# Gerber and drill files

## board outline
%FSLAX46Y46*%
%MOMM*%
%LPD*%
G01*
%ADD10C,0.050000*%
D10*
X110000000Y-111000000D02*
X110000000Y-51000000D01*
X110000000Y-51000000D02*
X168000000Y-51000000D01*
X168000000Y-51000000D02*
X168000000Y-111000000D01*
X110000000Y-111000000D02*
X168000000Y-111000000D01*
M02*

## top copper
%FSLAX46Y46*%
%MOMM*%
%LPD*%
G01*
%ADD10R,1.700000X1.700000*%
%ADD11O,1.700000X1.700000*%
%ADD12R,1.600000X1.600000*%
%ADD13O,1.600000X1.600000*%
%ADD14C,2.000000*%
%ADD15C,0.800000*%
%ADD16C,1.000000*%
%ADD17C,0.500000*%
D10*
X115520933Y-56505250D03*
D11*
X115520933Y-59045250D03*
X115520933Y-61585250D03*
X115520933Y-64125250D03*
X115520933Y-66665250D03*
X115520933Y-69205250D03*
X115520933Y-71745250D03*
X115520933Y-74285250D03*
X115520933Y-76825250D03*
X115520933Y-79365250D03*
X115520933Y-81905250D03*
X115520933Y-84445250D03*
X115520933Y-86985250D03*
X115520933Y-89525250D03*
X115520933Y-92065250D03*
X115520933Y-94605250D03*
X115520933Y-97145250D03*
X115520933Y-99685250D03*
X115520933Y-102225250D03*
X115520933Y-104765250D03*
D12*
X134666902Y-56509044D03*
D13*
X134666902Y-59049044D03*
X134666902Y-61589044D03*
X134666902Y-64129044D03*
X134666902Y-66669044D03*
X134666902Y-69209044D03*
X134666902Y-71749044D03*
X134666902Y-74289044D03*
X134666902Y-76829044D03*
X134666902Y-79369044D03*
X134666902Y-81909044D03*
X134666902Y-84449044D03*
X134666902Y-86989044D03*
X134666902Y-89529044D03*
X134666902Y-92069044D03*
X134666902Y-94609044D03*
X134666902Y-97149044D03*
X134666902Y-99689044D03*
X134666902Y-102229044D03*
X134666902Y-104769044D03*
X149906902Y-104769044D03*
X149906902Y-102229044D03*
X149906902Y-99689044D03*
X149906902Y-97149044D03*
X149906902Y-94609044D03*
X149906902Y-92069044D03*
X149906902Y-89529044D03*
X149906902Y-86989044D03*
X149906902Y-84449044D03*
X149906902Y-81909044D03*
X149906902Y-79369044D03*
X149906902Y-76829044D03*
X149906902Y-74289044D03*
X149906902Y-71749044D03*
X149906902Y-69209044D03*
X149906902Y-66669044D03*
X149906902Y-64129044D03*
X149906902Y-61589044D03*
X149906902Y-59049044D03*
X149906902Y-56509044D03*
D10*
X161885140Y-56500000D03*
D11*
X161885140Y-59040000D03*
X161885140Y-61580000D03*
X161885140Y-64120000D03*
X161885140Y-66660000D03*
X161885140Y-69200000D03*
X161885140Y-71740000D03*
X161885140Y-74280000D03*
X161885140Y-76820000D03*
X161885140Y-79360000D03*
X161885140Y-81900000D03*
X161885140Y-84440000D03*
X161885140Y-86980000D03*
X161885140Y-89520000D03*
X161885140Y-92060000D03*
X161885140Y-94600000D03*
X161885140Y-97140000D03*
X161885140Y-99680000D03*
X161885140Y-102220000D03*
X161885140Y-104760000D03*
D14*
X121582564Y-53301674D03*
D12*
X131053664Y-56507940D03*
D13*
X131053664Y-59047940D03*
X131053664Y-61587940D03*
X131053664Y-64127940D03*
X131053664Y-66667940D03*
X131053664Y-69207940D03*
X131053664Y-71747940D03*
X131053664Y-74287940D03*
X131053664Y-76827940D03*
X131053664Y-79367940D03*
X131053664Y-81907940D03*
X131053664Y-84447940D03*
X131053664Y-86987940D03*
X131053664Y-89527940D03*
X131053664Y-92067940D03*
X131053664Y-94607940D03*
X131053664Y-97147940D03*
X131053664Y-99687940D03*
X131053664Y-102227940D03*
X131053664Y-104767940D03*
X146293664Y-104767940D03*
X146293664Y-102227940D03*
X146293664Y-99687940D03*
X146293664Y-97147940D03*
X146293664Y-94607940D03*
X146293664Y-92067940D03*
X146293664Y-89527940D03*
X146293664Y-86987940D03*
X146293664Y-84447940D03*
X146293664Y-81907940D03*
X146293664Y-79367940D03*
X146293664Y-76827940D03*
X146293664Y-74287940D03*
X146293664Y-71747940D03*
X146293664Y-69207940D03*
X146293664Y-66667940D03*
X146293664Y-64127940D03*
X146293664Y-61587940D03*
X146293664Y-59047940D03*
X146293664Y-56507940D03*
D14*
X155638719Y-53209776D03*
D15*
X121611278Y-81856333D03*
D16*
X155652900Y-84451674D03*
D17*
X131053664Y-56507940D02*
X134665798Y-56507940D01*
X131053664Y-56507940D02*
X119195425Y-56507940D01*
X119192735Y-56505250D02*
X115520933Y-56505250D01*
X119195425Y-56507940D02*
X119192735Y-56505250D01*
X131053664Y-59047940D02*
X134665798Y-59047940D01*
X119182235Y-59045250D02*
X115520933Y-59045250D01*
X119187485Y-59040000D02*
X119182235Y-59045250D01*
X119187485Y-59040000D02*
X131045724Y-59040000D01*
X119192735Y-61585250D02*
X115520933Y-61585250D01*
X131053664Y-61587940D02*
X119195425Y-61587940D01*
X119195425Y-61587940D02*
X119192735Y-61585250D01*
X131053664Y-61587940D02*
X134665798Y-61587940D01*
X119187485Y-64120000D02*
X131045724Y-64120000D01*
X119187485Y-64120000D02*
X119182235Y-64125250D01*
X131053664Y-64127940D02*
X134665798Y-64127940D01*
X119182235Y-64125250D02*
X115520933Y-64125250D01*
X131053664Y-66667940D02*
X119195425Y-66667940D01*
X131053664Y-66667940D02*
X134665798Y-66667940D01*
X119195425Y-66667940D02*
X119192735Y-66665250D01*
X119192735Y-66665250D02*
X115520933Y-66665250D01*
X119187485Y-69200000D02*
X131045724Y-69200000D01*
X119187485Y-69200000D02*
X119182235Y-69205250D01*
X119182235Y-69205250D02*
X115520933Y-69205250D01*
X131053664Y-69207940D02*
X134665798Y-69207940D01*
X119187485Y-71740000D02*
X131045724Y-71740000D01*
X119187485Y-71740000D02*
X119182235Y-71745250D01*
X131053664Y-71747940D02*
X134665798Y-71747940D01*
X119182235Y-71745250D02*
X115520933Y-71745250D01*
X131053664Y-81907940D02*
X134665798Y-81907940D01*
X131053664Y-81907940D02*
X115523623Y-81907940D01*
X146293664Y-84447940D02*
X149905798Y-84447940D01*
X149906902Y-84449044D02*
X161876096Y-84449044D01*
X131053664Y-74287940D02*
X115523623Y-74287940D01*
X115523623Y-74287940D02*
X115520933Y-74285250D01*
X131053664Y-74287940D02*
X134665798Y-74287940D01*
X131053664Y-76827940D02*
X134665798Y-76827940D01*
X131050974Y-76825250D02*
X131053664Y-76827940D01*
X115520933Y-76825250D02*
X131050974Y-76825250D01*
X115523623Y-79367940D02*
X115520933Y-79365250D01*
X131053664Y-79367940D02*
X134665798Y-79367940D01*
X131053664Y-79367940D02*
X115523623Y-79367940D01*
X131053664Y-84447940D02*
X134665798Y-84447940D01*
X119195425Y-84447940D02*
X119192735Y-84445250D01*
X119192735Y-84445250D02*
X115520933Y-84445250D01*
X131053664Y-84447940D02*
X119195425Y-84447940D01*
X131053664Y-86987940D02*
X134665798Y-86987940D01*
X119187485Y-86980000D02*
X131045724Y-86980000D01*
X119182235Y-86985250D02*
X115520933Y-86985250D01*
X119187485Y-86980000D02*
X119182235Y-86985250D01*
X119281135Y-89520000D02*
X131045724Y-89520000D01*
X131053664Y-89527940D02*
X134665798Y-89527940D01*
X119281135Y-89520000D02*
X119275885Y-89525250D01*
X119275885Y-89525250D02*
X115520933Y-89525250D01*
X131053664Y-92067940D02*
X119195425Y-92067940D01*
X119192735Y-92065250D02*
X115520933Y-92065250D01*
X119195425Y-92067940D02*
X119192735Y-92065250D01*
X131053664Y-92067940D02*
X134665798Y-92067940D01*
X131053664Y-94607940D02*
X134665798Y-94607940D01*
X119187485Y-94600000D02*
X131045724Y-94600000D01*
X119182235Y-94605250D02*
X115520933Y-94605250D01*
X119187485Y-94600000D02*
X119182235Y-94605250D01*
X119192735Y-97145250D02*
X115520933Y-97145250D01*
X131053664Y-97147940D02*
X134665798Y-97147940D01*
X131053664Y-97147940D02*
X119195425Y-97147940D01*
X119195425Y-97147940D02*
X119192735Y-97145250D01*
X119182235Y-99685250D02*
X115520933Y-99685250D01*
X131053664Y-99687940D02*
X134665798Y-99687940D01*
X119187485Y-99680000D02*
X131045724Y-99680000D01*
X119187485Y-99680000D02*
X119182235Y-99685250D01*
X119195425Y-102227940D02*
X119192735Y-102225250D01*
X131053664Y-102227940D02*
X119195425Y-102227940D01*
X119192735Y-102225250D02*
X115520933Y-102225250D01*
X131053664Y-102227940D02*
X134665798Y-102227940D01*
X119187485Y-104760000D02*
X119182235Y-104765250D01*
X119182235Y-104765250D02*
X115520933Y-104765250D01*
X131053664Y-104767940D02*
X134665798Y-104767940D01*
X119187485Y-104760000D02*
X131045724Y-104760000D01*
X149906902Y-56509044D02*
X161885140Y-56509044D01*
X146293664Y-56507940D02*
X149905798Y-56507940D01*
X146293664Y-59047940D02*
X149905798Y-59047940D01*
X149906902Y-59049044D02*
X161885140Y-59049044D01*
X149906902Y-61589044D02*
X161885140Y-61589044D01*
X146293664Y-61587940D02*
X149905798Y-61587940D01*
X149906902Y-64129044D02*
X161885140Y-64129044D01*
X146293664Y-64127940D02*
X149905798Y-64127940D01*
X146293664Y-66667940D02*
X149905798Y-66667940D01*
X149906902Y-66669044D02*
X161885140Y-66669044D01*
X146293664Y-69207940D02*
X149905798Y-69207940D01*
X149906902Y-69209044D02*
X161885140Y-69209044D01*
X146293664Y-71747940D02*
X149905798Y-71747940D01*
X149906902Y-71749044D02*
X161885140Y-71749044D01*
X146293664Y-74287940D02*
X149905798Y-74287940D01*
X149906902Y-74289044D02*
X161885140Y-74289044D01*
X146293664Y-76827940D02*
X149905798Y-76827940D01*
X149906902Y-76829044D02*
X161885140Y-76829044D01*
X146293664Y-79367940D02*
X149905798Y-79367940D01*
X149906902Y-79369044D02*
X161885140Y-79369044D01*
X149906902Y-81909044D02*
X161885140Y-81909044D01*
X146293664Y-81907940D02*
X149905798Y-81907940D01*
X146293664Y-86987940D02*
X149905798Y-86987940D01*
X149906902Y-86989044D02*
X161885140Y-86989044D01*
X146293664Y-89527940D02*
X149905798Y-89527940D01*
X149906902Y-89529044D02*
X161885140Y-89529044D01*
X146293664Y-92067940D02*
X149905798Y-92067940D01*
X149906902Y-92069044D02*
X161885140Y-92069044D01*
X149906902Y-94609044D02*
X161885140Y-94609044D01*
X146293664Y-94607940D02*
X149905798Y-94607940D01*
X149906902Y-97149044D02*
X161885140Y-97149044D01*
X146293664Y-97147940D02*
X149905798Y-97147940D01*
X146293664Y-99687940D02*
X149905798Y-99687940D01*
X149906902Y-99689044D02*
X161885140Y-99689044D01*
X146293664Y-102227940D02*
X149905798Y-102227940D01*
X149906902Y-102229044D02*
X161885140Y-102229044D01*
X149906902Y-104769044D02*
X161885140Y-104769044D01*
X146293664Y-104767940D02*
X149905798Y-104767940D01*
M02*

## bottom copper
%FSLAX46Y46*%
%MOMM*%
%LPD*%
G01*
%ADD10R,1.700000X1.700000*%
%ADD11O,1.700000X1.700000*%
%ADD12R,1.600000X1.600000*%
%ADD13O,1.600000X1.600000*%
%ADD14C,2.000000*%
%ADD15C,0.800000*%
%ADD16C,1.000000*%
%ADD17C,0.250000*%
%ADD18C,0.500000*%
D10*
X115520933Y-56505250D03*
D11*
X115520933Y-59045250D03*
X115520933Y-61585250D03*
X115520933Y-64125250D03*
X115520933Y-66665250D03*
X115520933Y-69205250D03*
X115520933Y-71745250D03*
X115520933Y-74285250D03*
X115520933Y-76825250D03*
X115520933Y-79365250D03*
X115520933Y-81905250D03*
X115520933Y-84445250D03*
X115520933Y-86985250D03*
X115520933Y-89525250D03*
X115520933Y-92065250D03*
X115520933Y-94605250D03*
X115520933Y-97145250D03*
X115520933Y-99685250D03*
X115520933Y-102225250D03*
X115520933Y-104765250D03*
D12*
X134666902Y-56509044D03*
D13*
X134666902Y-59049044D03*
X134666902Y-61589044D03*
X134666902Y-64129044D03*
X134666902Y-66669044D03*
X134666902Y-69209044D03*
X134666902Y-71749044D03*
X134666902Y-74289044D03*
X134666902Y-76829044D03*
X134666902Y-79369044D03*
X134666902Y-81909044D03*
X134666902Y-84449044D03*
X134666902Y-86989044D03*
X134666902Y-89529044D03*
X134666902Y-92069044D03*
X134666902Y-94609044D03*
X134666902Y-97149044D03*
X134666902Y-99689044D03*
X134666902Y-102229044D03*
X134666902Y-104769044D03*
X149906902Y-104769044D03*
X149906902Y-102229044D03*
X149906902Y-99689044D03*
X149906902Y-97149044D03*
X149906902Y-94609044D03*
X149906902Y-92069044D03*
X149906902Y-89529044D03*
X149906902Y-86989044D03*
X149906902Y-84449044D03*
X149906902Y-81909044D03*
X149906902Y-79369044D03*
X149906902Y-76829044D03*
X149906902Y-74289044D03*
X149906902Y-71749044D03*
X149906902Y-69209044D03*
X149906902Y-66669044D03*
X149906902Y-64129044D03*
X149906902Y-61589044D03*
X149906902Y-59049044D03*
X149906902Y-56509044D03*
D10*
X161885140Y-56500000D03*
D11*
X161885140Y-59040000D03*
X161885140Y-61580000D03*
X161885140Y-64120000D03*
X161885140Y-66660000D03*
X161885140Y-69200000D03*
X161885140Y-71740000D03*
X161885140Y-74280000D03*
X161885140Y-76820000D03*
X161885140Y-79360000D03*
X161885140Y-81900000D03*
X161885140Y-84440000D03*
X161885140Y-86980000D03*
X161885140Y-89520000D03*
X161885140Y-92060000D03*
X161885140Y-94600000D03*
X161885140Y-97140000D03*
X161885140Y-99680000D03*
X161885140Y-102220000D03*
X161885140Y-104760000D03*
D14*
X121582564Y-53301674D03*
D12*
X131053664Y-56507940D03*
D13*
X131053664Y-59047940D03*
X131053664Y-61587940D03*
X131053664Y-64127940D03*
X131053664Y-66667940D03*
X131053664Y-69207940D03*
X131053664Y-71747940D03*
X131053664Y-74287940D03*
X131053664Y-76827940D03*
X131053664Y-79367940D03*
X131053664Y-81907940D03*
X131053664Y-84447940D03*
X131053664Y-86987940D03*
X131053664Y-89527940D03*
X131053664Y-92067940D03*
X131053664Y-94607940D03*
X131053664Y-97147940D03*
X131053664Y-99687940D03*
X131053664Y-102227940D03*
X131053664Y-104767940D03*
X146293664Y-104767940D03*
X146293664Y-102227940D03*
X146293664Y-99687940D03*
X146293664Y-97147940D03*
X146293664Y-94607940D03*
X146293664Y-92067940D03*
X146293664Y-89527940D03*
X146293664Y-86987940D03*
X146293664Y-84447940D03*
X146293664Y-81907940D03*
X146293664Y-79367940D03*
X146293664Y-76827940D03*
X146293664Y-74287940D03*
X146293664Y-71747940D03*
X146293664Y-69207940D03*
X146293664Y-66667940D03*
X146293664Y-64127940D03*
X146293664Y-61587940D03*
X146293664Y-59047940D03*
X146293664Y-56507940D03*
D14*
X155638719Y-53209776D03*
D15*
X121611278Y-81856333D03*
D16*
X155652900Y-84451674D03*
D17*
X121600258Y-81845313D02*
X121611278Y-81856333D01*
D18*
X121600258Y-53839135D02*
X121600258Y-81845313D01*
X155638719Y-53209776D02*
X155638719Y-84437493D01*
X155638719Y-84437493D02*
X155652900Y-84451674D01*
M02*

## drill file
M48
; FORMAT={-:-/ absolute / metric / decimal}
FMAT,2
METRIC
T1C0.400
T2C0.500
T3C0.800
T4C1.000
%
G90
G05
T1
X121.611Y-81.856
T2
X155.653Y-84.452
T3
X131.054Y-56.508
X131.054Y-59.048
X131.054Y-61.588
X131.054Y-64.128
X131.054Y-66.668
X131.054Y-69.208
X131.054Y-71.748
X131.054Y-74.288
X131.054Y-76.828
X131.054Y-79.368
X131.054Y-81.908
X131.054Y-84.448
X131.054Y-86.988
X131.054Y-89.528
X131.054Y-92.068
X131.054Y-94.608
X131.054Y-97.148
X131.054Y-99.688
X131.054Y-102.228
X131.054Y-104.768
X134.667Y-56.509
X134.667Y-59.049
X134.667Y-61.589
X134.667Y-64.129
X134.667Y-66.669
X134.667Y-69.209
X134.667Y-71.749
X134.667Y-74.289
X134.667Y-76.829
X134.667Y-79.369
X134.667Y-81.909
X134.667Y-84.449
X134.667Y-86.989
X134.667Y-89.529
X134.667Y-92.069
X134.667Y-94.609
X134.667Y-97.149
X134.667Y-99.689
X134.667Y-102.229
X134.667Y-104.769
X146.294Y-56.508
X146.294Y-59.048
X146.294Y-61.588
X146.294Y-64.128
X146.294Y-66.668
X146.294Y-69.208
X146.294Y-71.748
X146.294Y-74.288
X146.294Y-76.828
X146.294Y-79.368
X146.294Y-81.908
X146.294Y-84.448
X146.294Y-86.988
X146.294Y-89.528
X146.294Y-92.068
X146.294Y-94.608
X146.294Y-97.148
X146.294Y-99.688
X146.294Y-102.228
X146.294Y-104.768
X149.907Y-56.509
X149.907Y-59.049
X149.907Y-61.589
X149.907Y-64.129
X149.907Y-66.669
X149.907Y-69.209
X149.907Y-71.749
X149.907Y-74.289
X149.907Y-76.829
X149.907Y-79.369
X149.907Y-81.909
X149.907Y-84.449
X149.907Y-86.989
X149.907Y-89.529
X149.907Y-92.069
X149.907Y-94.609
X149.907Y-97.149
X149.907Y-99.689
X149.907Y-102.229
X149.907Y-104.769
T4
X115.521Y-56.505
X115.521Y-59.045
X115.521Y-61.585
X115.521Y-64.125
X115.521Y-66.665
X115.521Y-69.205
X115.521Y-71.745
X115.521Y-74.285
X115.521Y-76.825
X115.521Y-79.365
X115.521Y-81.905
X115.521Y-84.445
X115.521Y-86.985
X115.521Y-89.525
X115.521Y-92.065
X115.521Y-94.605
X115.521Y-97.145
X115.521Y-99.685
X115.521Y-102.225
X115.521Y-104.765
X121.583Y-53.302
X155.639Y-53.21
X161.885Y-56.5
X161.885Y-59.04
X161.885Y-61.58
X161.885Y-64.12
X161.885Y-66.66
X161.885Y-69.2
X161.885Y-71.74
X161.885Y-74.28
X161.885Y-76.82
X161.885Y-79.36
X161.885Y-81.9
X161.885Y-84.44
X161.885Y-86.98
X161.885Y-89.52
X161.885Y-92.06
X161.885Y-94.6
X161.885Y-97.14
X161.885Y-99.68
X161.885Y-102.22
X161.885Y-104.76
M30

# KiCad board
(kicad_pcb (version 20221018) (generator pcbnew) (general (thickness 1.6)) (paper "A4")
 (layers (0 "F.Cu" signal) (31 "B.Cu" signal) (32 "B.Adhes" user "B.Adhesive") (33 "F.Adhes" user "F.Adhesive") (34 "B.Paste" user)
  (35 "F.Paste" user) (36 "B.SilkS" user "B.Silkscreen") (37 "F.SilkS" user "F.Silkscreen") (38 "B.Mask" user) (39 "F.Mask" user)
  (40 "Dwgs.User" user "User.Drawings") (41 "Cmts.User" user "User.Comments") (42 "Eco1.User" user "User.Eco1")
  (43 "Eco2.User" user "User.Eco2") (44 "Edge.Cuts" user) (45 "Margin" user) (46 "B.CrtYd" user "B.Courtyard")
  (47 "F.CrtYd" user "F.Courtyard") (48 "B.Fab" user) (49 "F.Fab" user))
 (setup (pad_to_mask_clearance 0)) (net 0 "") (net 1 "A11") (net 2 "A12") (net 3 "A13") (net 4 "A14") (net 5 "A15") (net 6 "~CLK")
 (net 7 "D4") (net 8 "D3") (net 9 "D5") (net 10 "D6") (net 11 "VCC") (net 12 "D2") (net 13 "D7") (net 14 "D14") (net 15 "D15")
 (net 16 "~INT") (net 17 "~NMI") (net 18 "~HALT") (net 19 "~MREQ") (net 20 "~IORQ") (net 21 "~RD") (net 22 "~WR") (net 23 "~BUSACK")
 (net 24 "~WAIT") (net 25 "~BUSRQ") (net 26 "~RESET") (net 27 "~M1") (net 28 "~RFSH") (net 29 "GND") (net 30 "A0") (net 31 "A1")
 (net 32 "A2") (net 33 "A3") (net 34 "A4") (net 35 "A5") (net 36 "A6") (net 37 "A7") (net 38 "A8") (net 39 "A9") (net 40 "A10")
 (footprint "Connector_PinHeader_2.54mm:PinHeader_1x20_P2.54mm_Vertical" (layer "F.Cu") (at 115.520933 56.50525)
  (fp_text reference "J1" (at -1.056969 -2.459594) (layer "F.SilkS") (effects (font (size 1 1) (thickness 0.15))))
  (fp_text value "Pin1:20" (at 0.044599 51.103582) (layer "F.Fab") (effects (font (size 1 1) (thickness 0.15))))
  (pad "1" thru_hole rect (at 0 0) (size 1.7 1.7) (drill 1) (layers "*.Cu" "*.Mask") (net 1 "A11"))
  (pad "2" thru_hole oval (at 0 2.54) (size 1.7 1.7) (drill 1) (layers "*.Cu" "*.Mask") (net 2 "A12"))
  (pad "3" thru_hole oval (at 0 5.08) (size 1.7 1.7) (drill 1) (layers "*.Cu" "*.Mask") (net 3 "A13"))
  (pad "4" thru_hole oval (at 0 7.62) (size 1.7 1.7) (drill 1) (layers "*.Cu" "*.Mask") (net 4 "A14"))
  (pad "5" thru_hole oval (at 0 10.16) (size 1.7 1.7) (drill 1) (layers "*.Cu" "*.Mask") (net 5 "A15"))
  (pad "6" thru_hole oval (at 0 12.7) (size 1.7 1.7) (drill 1) (layers "*.Cu" "*.Mask") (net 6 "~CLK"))
  (pad "7" thru_hole oval (at 0 15.24) (size 1.7 1.7) (drill 1) (layers "*.Cu" "*.Mask") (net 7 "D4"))
  (pad "8" thru_hole oval (at 0 17.78) (size 1.7 1.7) (drill 1) (layers "*.Cu" "*.Mask") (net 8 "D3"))
  (pad "9" thru_hole oval (at 0 20.32) (size 1.7 1.7) (drill 1) (layers "*.Cu" "*.Mask") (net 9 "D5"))
  (pad "10" thru_hole oval (at 0 22.86) (size 1.7 1.7) (drill 1) (layers "*.Cu" "*.Mask") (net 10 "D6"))
  (pad "11" thru_hole oval (at 0 25.4) (size 1.7 1.7) (drill 1) (layers "*.Cu" "*.Mask") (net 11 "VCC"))
  (pad "12" thru_hole oval (at 0 27.94) (size 1.7 1.7) (drill 1) (layers "*.Cu" "*.Mask") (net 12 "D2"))
  (pad "13" thru_hole oval (at 0 30.48) (size 1.7 1.7) (drill 1) (layers "*.Cu" "*.Mask") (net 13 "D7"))
  (pad "14" thru_hole oval (at 0 33.02) (size 1.7 1.7) (drill 1) (layers "*.Cu" "*.Mask") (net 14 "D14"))
  (pad "15" thru_hole oval (at 0 35.56) (size 1.7 1.7) (drill 1) (layers "*.Cu" "*.Mask") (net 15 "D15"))
  (pad "16" thru_hole oval (at 0 38.1) (size 1.7 1.7) (drill 1) (layers "*.Cu" "*.Mask") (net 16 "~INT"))
  (pad "17" thru_hole oval (at 0 40.64) (size 1.7 1.7) (drill 1) (layers "*.Cu" "*.Mask") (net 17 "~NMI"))
  (pad "18" thru_hole oval (at 0 43.18) (size 1.7 1.7) (drill 1) (layers "*.Cu" "*.Mask") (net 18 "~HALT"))
  (pad "19" thru_hole oval (at 0 45.72) (size 1.7 1.7) (drill 1) (layers "*.Cu" "*.Mask") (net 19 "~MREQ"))
  (pad "20" thru_hole oval (at 0 48.26) (size 1.7 1.7) (drill 1) (layers "*.Cu" "*.Mask") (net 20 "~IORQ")))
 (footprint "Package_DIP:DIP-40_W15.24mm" (layer "F.Cu") (at 134.666902 56.509044)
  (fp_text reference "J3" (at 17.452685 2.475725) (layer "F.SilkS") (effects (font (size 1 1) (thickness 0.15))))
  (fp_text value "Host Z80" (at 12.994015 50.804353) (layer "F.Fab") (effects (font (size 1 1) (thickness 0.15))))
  (pad "1" thru_hole rect (at 0 0) (size 1.6 1.6) (drill 0.8) (layers "*.Cu" "*.Mask") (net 1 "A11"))
  (pad "2" thru_hole oval (at 0 2.54) (size 1.6 1.6) (drill 0.8) (layers "*.Cu" "*.Mask") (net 2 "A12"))
  (pad "3" thru_hole oval (at 0 5.08) (size 1.6 1.6) (drill 0.8) (layers "*.Cu" "*.Mask") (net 3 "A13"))
  (pad "4" thru_hole oval (at 0 7.62) (size 1.6 1.6) (drill 0.8) (layers "*.Cu" "*.Mask") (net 4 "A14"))
  (pad "5" thru_hole oval (at 0 10.16) (size 1.6 1.6) (drill 0.8) (layers "*.Cu" "*.Mask") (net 5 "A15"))
  (pad "6" thru_hole oval (at 0 12.7) (size 1.6 1.6) (drill 0.8) (layers "*.Cu" "*.Mask") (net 6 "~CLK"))
  (pad "7" thru_hole oval (at 0 15.24) (size 1.6 1.6) (drill 0.8) (layers "*.Cu" "*.Mask") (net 7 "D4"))
  (pad "8" thru_hole oval (at 0 17.78) (size 1.6 1.6) (drill 0.8) (layers "*.Cu" "*.Mask") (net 8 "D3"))
  (pad "9" thru_hole oval (at 0 20.32) (size 1.6 1.6) (drill 0.8) (layers "*.Cu" "*.Mask") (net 9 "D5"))
  (pad "10" thru_hole oval (at 0 22.86) (size 1.6 1.6) (drill 0.8) (layers "*.Cu" "*.Mask") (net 10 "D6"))
  (pad "11" thru_hole oval (at 0 25.4) (size 1.6 1.6) (drill 0.8) (layers "*.Cu" "*.Mask") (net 11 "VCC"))
  (pad "12" thru_hole oval (at 0 27.94) (size 1.6 1.6) (drill 0.8) (layers "*.Cu" "*.Mask") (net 12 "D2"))
  (pad "13" thru_hole oval (at 0 30.48) (size 1.6 1.6) (drill 0.8) (layers "*.Cu" "*.Mask") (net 13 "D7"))
  (pad "14" thru_hole oval (at 0 33.02) (size 1.6 1.6) (drill 0.8) (layers "*.Cu" "*.Mask") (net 14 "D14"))
  (pad "15" thru_hole oval (at 0 35.56) (size 1.6 1.6) (drill 0.8) (layers "*.Cu" "*.Mask") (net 15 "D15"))
  (pad "16" thru_hole oval (at 0 38.1) (size 1.6 1.6) (drill 0.8) (layers "*.Cu" "*.Mask") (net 16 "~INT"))
  (pad "17" thru_hole oval (at 0 40.64) (size 1.6 1.6) (drill 0.8) (layers "*.Cu" "*.Mask") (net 17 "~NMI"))
  (pad "18" thru_hole oval (at 0 43.18) (size 1.6 1.6) (drill 0.8) (layers "*.Cu" "*.Mask") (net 18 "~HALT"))
  (pad "19" thru_hole oval (at 0 45.72) (size 1.6 1.6) (drill 0.8) (layers "*.Cu" "*.Mask") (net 19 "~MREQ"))
  (pad "20" thru_hole oval (at 0 48.26) (size 1.6 1.6) (drill 0.8) (layers "*.Cu" "*.Mask") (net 20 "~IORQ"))
  (pad "21" thru_hole oval (at 15.24 48.26) (size 1.6 1.6) (drill 0.8) (layers "*.Cu" "*.Mask") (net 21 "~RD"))
  (pad "22" thru_hole oval (at 15.24 45.72) (size 1.6 1.6) (drill 0.8) (layers "*.Cu" "*.Mask") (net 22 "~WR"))
  (pad "23" thru_hole oval (at 15.24 43.18) (size 1.6 1.6) (drill 0.8) (layers "*.Cu" "*.Mask") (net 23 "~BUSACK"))
  (pad "24" thru_hole oval (at 15.24 40.64) (size 1.6 1.6) (drill 0.8) (layers "*.Cu" "*.Mask") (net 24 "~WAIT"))
  (pad "25" thru_hole oval (at 15.24 38.1) (size 1.6 1.6) (drill 0.8) (layers "*.Cu" "*.Mask") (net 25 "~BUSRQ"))
  (pad "26" thru_hole oval (at 15.24 35.56) (size 1.6 1.6) (drill 0.8) (layers "*.Cu" "*.Mask") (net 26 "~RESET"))
  (pad "27" thru_hole oval (at 15.24 33.02) (size 1.6 1.6) (drill 0.8) (layers "*.Cu" "*.Mask") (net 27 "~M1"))
  (pad "28" thru_hole oval (at 15.24 30.48) (size 1.6 1.6) (drill 0.8) (layers "*.Cu" "*.Mask") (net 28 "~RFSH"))
  (pad "29" thru_hole oval (at 15.24 27.94) (size 1.6 1.6) (drill 0.8) (layers "*.Cu" "*.Mask") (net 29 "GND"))
  (pad "30" thru_hole oval (at 15.24 25.4) (size 1.6 1.6) (drill 0.8) (layers "*.Cu" "*.Mask") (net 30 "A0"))
  (pad "31" thru_hole oval (at 15.24 22.86) (size 1.6 1.6) (drill 0.8) (layers "*.Cu" "*.Mask") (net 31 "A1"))
  (pad "32" thru_hole oval (at 15.24 20.32) (size 1.6 1.6) (drill 0.8) (layers "*.Cu" "*.Mask") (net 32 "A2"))
  (pad "33" thru_hole oval (at 15.24 17.78) (size 1.6 1.6) (drill 0.8) (layers "*.Cu" "*.Mask") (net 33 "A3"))
  (pad "34" thru_hole oval (at 15.24 15.24) (size 1.6 1.6) (drill 0.8) (layers "*.Cu" "*.Mask") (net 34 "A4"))
  (pad "35" thru_hole oval (at 15.24 12.7) (size 1.6 1.6) (drill 0.8) (layers "*.Cu" "*.Mask") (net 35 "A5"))
  (pad "36" thru_hole oval (at 15.24 10.16) (size 1.6 1.6) (drill 0.8) (layers "*.Cu" "*.Mask") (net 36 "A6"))
  (pad "37" thru_hole oval (at 15.24 7.62) (size 1.6 1.6) (drill 0.8) (layers "*.Cu" "*.Mask") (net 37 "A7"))
  (pad "38" thru_hole oval (at 15.24 5.08) (size 1.6 1.6) (drill 0.8) (layers "*.Cu" "*.Mask") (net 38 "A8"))
  (pad "39" thru_hole oval (at 15.24 2.54) (size 1.6 1.6) (drill 0.8) (layers "*.Cu" "*.Mask") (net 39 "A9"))
  (pad "40" thru_hole oval (at 15.24 0) (size 1.6 1.6) (drill 0.8) (layers "*.Cu" "*.Mask") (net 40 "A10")))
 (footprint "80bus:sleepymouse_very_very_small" (layer "F.Cu") (at 140.734198 96.369357 -90)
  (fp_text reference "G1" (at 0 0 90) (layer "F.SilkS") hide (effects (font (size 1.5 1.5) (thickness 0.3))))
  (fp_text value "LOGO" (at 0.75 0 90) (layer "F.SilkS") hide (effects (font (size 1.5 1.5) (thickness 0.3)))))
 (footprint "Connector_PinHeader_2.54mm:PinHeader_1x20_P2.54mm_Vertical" (layer "F.Cu") (at 161.88514 56.5)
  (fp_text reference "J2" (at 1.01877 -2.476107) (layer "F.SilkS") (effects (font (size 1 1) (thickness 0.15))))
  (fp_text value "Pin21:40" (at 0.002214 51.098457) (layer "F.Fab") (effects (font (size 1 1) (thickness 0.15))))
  (pad "1" thru_hole rect (at 0 0) (size 1.7 1.7) (drill 1) (layers "*.Cu" "*.Mask") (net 40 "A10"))
  (pad "2" thru_hole oval (at 0 2.54) (size 1.7 1.7) (drill 1) (layers "*.Cu" "*.Mask") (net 39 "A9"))
  (pad "3" thru_hole oval (at 0 5.08) (size 1.7 1.7) (drill 1) (layers "*.Cu" "*.Mask") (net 38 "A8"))
  (pad "4" thru_hole oval (at 0 7.62) (size 1.7 1.7) (drill 1) (layers "*.Cu" "*.Mask") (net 37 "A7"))
  (pad "5" thru_hole oval (at 0 10.16) (size 1.7 1.7) (drill 1) (layers "*.Cu" "*.Mask") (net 36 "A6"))
  (pad "6" thru_hole oval (at 0 12.7) (size 1.7 1.7) (drill 1) (layers "*.Cu" "*.Mask") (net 35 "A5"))
  (pad "7" thru_hole oval (at 0 15.24) (size 1.7 1.7) (drill 1) (layers "*.Cu" "*.Mask") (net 34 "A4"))
  (pad "8" thru_hole oval (at 0 17.78) (size 1.7 1.7) (drill 1) (layers "*.Cu" "*.Mask") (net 33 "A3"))
  (pad "9" thru_hole oval (at 0 20.32) (size 1.7 1.7) (drill 1) (layers "*.Cu" "*.Mask") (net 32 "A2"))
  (pad "10" thru_hole oval (at 0 22.86) (size 1.7 1.7) (drill 1) (layers "*.Cu" "*.Mask") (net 31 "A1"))
  (pad "11" thru_hole oval (at 0 25.4) (size 1.7 1.7) (drill 1) (layers "*.Cu" "*.Mask") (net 30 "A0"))
  (pad "12" thru_hole oval (at 0 27.94) (size 1.7 1.7) (drill 1) (layers "*.Cu" "*.Mask") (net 29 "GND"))
  (pad "13" thru_hole oval (at 0 30.48) (size 1.7 1.7) (drill 1) (layers "*.Cu" "*.Mask") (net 28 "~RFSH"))
  (pad "14" thru_hole oval (at 0 33.02) (size 1.7 1.7) (drill 1) (layers "*.Cu" "*.Mask") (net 27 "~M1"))
  (pad "15" thru_hole oval (at 0 35.56) (size 1.7 1.7) (drill 1) (layers "*.Cu" "*.Mask") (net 26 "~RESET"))
  (pad "16" thru_hole oval (at 0 38.1) (size 1.7 1.7) (drill 1) (layers "*.Cu" "*.Mask") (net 25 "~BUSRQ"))
  (pad "17" thru_hole oval (at 0 40.64) (size 1.7 1.7) (drill 1) (layers "*.Cu" "*.Mask") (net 24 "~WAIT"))
  (pad "18" thru_hole oval (at 0 43.18) (size 1.7 1.7) (drill 1) (layers "*.Cu" "*.Mask") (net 23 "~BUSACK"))
  (pad "19" thru_hole oval (at 0 45.72) (size 1.7 1.7) (drill 1) (layers "*.Cu" "*.Mask") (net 22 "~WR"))
  (pad "20" thru_hole oval (at 0 48.26) (size 1.7 1.7) (drill 1) (layers "*.Cu" "*.Mask") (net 21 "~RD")))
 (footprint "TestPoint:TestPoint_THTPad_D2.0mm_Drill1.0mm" (layer "F.Cu") (at 121.582564 53.301674)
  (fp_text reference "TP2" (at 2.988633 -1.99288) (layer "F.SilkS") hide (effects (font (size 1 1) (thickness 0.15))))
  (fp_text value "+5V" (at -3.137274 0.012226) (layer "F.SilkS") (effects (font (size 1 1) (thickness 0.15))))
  (pad "1" thru_hole circle (at 0 0) (size 2 2) (drill 1) (layers "*.Cu" "*.Mask") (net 11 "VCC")))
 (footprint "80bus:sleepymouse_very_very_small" (layer "F.Cu") (at 140.5903 65.359205 -90)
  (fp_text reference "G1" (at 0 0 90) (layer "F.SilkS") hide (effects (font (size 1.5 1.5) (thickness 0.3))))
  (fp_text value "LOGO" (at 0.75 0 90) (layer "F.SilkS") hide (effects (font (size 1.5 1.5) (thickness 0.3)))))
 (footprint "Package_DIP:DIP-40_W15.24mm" (layer "F.Cu") (at 131.053664 56.50794)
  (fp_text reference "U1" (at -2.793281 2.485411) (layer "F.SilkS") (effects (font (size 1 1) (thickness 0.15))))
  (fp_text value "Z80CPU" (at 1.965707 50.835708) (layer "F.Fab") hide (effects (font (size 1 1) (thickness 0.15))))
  (pad "1" thru_hole rect (at 0 0) (size 1.6 1.6) (drill 0.8) (layers "*.Cu" "*.Mask") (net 1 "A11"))
  (pad "2" thru_hole oval (at 0 2.54) (size 1.6 1.6) (drill 0.8) (layers "*.Cu" "*.Mask") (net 2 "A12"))
  (pad "3" thru_hole oval (at 0 5.08) (size 1.6 1.6) (drill 0.8) (layers "*.Cu" "*.Mask") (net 3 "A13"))
  (pad "4" thru_hole oval (at 0 7.62) (size 1.6 1.6) (drill 0.8) (layers "*.Cu" "*.Mask") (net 4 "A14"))
  (pad "5" thru_hole oval (at 0 10.16) (size 1.6 1.6) (drill 0.8) (layers "*.Cu" "*.Mask") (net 5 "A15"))
  (pad "6" thru_hole oval (at 0 12.7) (size 1.6 1.6) (drill 0.8) (layers "*.Cu" "*.Mask") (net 6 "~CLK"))
  (pad "7" thru_hole oval (at 0 15.24) (size 1.6 1.6) (drill 0.8) (layers "*.Cu" "*.Mask") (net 7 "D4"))
  (pad "8" thru_hole oval (at 0 17.78) (size 1.6 1.6) (drill 0.8) (layers "*.Cu" "*.Mask") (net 8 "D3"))
  (pad "9" thru_hole oval (at 0 20.32) (size 1.6 1.6) (drill 0.8) (layers "*.Cu" "*.Mask") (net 9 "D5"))
  (pad "10" thru_hole oval (at 0 22.86) (size 1.6 1.6) (drill 0.8) (layers "*.Cu" "*.Mask") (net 10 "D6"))
  (pad "11" thru_hole oval (at 0 25.4) (size 1.6 1.6) (drill 0.8) (layers "*.Cu" "*.Mask") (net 11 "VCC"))
  (pad "12" thru_hole oval (at 0 27.94) (size 1.6 1.6) (drill 0.8) (layers "*.Cu" "*.Mask") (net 12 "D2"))
  (pad "13" thru_hole oval (at 0 30.48) (size 1.6 1.6) (drill 0.8) (layers "*.Cu" "*.Mask") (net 13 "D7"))
  (pad "14" thru_hole oval (at 0 33.02) (size 1.6 1.6) (drill 0.8) (layers "*.Cu" "*.Mask") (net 14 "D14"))
  (pad "15" thru_hole oval (at 0 35.56) (size 1.6 1.6) (drill 0.8) (layers "*.Cu" "*.Mask") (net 15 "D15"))
  (pad "16" thru_hole oval (at 0 38.1) (size 1.6 1.6) (drill 0.8) (layers "*.Cu" "*.Mask") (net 16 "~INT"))
  (pad "17" thru_hole oval (at 0 40.64) (size 1.6 1.6) (drill 0.8) (layers "*.Cu" "*.Mask") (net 17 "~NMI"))
  (pad "18" thru_hole oval (at 0 43.18) (size 1.6 1.6) (drill 0.8) (layers "*.Cu" "*.Mask") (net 18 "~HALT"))
  (pad "19" thru_hole oval (at 0 45.72) (size 1.6 1.6) (drill 0.8) (layers "*.Cu" "*.Mask") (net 19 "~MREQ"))
  (pad "20" thru_hole oval (at 0 48.26) (size 1.6 1.6) (drill 0.8) (layers "*.Cu" "*.Mask") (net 20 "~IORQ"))
  (pad "21" thru_hole oval (at 15.24 48.26) (size 1.6 1.6) (drill 0.8) (layers "*.Cu" "*.Mask") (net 21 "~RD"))
  (pad "22" thru_hole oval (at 15.24 45.72) (size 1.6 1.6) (drill 0.8) (layers "*.Cu" "*.Mask") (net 22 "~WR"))
  (pad "23" thru_hole oval (at 15.24 43.18) (size 1.6 1.6) (drill 0.8) (layers "*.Cu" "*.Mask") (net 23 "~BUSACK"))
  (pad "24" thru_hole oval (at 15.24 40.64) (size 1.6 1.6) (drill 0.8) (layers "*.Cu" "*.Mask") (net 24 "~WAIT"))
  (pad "25" thru_hole oval (at 15.24 38.1) (size 1.6 1.6) (drill 0.8) (layers "*.Cu" "*.Mask") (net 25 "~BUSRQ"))
  (pad "26" thru_hole oval (at 15.24 35.56) (size 1.6 1.6) (drill 0.8) (layers "*.Cu" "*.Mask") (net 26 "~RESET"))
  (pad "27" thru_hole oval (at 15.24 33.02) (size 1.6 1.6) (drill 0.8) (layers "*.Cu" "*.Mask") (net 27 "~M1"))
  (pad "28" thru_hole oval (at 15.24 30.48) (size 1.6 1.6) (drill 0.8) (layers "*.Cu" "*.Mask") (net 28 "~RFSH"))
  (pad "29" thru_hole oval (at 15.24 27.94) (size 1.6 1.6) (drill 0.8) (layers "*.Cu" "*.Mask") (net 29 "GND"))
  (pad "30" thru_hole oval (at 15.24 25.4) (size 1.6 1.6) (drill 0.8) (layers "*.Cu" "*.Mask") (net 30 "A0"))
  (pad "31" thru_hole oval (at 15.24 22.86) (size 1.6 1.6) (drill 0.8) (layers "*.Cu" "*.Mask") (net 31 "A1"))
  (pad "32" thru_hole oval (at 15.24 20.32) (size 1.6 1.6) (drill 0.8) (layers "*.Cu" "*.Mask") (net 32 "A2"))
  (pad "33" thru_hole oval (at 15.24 17.78) (size 1.6 1.6) (drill 0.8) (layers "*.Cu" "*.Mask") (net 33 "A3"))
  (pad "34" thru_hole oval (at 15.24 15.24) (size 1.6 1.6) (drill 0.8) (layers "*.Cu" "*.Mask") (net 34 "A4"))
  (pad "35" thru_hole oval (at 15.24 12.7) (size 1.6 1.6) (drill 0.8) (layers "*.Cu" "*.Mask") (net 35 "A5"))
  (pad "36" thru_hole oval (at 15.24 10.16) (size 1.6 1.6) (drill 0.8) (layers "*.Cu" "*.Mask") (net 36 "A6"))
  (pad "37" thru_hole oval (at 15.24 7.62) (size 1.6 1.6) (drill 0.8) (layers "*.Cu" "*.Mask") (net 37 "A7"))
  (pad "38" thru_hole oval (at 15.24 5.08) (size 1.6 1.6) (drill 0.8) (layers "*.Cu" "*.Mask") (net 38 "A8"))
  (pad "39" thru_hole oval (at 15.24 2.54) (size 1.6 1.6) (drill 0.8) (layers "*.Cu" "*.Mask") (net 39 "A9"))
  (pad "40" thru_hole oval (at 15.24 0) (size 1.6 1.6) (drill 0.8) (layers "*.Cu" "*.Mask") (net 40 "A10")))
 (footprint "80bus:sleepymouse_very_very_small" (layer "F.Cu") (at 140.481043 80.489878 -90)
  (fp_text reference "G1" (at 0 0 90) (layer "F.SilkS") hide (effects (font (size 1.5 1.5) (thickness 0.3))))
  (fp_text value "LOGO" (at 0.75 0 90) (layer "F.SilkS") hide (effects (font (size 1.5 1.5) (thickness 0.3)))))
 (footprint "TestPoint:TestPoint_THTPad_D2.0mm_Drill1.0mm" (layer "F.Cu") (at 155.638719 53.209776)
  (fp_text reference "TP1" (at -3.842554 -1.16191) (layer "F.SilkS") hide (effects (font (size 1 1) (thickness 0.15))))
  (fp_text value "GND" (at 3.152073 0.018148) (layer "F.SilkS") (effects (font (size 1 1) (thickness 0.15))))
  (pad "1" thru_hole circle (at 0 0) (size 2 2) (drill 1) (layers "*.Cu" "*.Mask") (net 29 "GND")))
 (gr_line (start 110 111) (end 110 51) (stroke (width 0.05) (type solid)) (layer "Edge.Cuts"))
 (gr_line (start 110 51) (end 168 51) (stroke (width 0.05) (type solid)) (layer "Edge.Cuts"))
 (gr_line (start 168 51) (end 168 111) (stroke (width 0.05) (type solid)) (layer "Edge.Cuts"))
 (gr_line (start 110 111) (end 168 111) (stroke (width 0.05) (type solid)) (layer "Edge.Cuts"))
 (segment (start 131.053664 56.50794) (end 134.665798 56.50794) (width 0.5) (layer "F.Cu") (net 1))
 (segment (start 131.053664 56.50794) (end 119.195425 56.50794) (width 0.5) (layer "F.Cu") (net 1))
 (segment (start 119.192735 56.50525) (end 115.520933 56.50525) (width 0.5) (layer "F.Cu") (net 1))
 (segment (start 119.195425 56.50794) (end 119.192735 56.50525) (width 0.5) (layer "F.Cu") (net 1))
 (segment (start 131.053664 59.04794) (end 134.665798 59.04794) (width 0.5) (layer "F.Cu") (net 2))
 (segment (start 119.182235 59.04525) (end 115.520933 59.04525) (width 0.5) (layer "F.Cu") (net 2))
 (segment (start 119.187485 59.04) (end 119.182235 59.04525) (width 0.5) (layer "F.Cu") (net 2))
 (segment (start 119.187485 59.04) (end 131.045724 59.04) (width 0.5) (layer "F.Cu") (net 2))
 (segment (start 119.192735 61.58525) (end 115.520933 61.58525) (width 0.5) (layer "F.Cu") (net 3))
 (segment (start 131.053664 61.58794) (end 119.195425 61.58794) (width 0.5) (layer "F.Cu") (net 3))
 (segment (start 119.195425 61.58794) (end 119.192735 61.58525) (width 0.5) (layer "F.Cu") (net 3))
 (segment (start 131.053664 61.58794) (end 134.665798 61.58794) (width 0.5) (layer "F.Cu") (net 3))
 (segment (start 119.187485 64.12) (end 131.045724 64.12) (width 0.5) (layer "F.Cu") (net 4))
 (segment (start 119.187485 64.12) (end 119.182235 64.12525) (width 0.5) (layer "F.Cu") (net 4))
 (segment (start 131.053664 64.12794) (end 134.665798 64.12794) (width 0.5) (layer "F.Cu") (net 4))
 (segment (start 119.182235 64.12525) (end 115.520933 64.12525) (width 0.5) (layer "F.Cu") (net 4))
 (segment (start 131.053664 66.66794) (end 119.195425 66.66794) (width 0.5) (layer "F.Cu") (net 5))
 (segment (start 131.053664 66.66794) (end 134.665798 66.66794) (width 0.5) (layer "F.Cu") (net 5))
 (segment (start 119.195425 66.66794) (end 119.192735 66.66525) (width 0.5) (layer "F.Cu") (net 5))
 (segment (start 119.192735 66.66525) (end 115.520933 66.66525) (width 0.5) (layer "F.Cu") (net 5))
 (segment (start 119.187485 69.2) (end 131.045724 69.2) (width 0.5) (layer "F.Cu") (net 6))
 (segment (start 119.187485 69.2) (end 119.182235 69.20525) (width 0.5) (layer "F.Cu") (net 6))
 (segment (start 119.182235 69.20525) (end 115.520933 69.20525) (width 0.5) (layer "F.Cu") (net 6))
 (segment (start 131.053664 69.20794) (end 134.665798 69.20794) (width 0.5) (layer "F.Cu") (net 6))
 (segment (start 119.187485 71.74) (end 131.045724 71.74) (width 0.5) (layer "F.Cu") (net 7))
 (segment (start 119.187485 71.74) (end 119.182235 71.74525) (width 0.5) (layer "F.Cu") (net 7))
 (segment (start 131.053664 71.74794) (end 134.665798 71.74794) (width 0.5) (layer "F.Cu") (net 7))
 (segment (start 119.182235 71.74525) (end 115.520933 71.74525) (width 0.5) (layer "F.Cu") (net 7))
 (segment (start 131.053664 81.90794) (end 134.665798 81.90794) (width 0.5) (layer "F.Cu") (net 11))
 (segment (start 131.053664 81.90794) (end 115.523623 81.90794) (width 0.5) (layer "F.Cu") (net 11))
 (via (at 121.611278 81.856333) (size 0.8) (drill 0.4) (layers "F.Cu" "B.Cu") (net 11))
 (segment (start 121.600258 81.845313) (end 121.611278 81.856333) (width 0.25) (layer "B.Cu") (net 11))
 (segment (start 121.600258 53.839135) (end 121.600258 81.845313) (width 0.5) (layer "B.Cu") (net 11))
 (segment (start 146.293664 84.44794) (end 149.905798 84.44794) (width 0.5) (layer "F.Cu") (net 29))
 (segment (start 149.906902 84.449044) (end 161.876096 84.449044) (width 0.5) (layer "F.Cu") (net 29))
 (via (at 155.6529 84.451674) (size 1) (drill 0.5) (layers "F.Cu" "B.Cu") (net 29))
 (segment (start 155.638719 53.209776) (end 155.638719 84.437493) (width 0.5) (layer "B.Cu") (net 29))
 (segment (start 155.638719 84.437493) (end 155.6529 84.451674) (width 0.5) (layer "B.Cu") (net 29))
 (segment (start 131.053664 74.28794) (end 115.523623 74.28794) (width 0.5) (layer "F.Cu") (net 8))
 (segment (start 115.523623 74.28794) (end 115.520933 74.28525) (width 0.5) (layer "F.Cu") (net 8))
 (segment (start 131.053664 74.28794) (end 134.665798 74.28794) (width 0.5) (layer "F.Cu") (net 8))
 (segment (start 131.053664 76.82794) (end 134.665798 76.82794) (width 0.5) (layer "F.Cu") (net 9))
 (segment (start 131.050974 76.82525) (end 131.053664 76.82794) (width 0.5) (layer "F.Cu") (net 9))
 (segment (start 115.520933 76.82525) (end 131.050974 76.82525) (width 0.5) (layer "F.Cu") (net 9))
 (segment (start 115.523623 79.36794) (end 115.520933 79.36525) (width 0.5) (layer "F.Cu") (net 10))
 (segment (start 131.053664 79.36794) (end 134.665798 79.36794) (width 0.5) (layer "F.Cu") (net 10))
 (segment (start 131.053664 79.36794) (end 115.523623 79.36794) (width 0.5) (layer "F.Cu") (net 10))
 (segment (start 131.053664 84.44794) (end 134.665798 84.44794) (width 0.5) (layer "F.Cu") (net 12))
 (segment (start 119.195425 84.44794) (end 119.192735 84.44525) (width 0.5) (layer "F.Cu") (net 12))
 (segment (start 119.192735 84.44525) (end 115.520933 84.44525) (width 0.5) (layer "F.Cu") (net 12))
 (segment (start 131.053664 84.44794) (end 119.195425 84.44794) (width 0.5) (layer "F.Cu") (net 12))
 (segment (start 131.053664 86.98794) (end 134.665798 86.98794) (width 0.5) (layer "F.Cu") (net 13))
 (segment (start 119.187485 86.98) (end 131.045724 86.98) (width 0.5) (layer "F.Cu") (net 13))
 (segment (start 119.182235 86.98525) (end 115.520933 86.98525) (width 0.5) (layer "F.Cu") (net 13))
 (segment (start 119.187485 86.98) (end 119.182235 86.98525) (width 0.5) (layer "F.Cu") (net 13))
 (segment (start 119.281135 89.52) (end 131.045724 89.52) (width 0.5) (layer "F.Cu") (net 14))
 (segment (start 131.053664 89.52794) (end 134.665798 89.52794) (width 0.5) (layer "F.Cu") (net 14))
 (segment (start 119.281135 89.52) (end 119.275885 89.52525) (width 0.5) (layer "F.Cu") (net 14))
 (segment (start 119.275885 89.52525) (end 115.520933 89.52525) (width 0.5) (layer "F.Cu") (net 14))
 (segment (start 131.053664 92.06794) (end 119.195425 92.06794) (width 0.5) (layer "F.Cu") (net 15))
 (segment (start 119.192735 92.06525) (end 115.520933 92.06525) (width 0.5) (layer "F.Cu") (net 15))
 (segment (start 119.195425 92.06794) (end 119.192735 92.06525) (width 0.5) (layer "F.Cu") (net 15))
 (segment (start 131.053664 92.06794) (end 134.665798 92.06794) (width 0.5) (layer "F.Cu") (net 15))
 (segment (start 131.053664 94.60794) (end 134.665798 94.60794) (width 0.5) (layer "F.Cu") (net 16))
 (segment (start 119.187485 94.6) (end 131.045724 94.6) (width 0.5) (layer "F.Cu") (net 16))
 (segment (start 119.182235 94.60525) (end 115.520933 94.60525) (width 0.5) (layer "F.Cu") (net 16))
 (segment (start 119.187485 94.6) (end 119.182235 94.60525) (width 0.5) (layer "F.Cu") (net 16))
 (segment (start 119.192735 97.14525) (end 115.520933 97.14525) (width 0.5) (layer "F.Cu") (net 17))
 (segment (start 131.053664 97.14794) (end 134.665798 97.14794) (width 0.5) (layer "F.Cu") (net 17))
 (segment (start 131.053664 97.14794) (end 119.195425 97.14794) (width 0.5) (layer "F.Cu") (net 17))
 (segment (start 119.195425 97.14794) (end 119.192735 97.14525) (width 0.5) (layer "F.Cu") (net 17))
 (segment (start 119.182235 99.68525) (end 115.520933 99.68525) (width 0.5) (layer "F.Cu") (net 18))
 (segment (start 131.053664 99.68794) (end 134.665798 99.68794) (width 0.5) (layer "F.Cu") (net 18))
 (segment (start 119.187485 99.68) (end 131.045724 99.68) (width 0.5) (layer "F.Cu") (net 18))
 (segment (start 119.187485 99.68) (end 119.182235 99.68525) (width 0.5) (layer "F.Cu") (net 18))
 (segment (start 119.195425 102.22794) (end 119.192735 102.22525) (width 0.5) (layer "F.Cu") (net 19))
 (segment (start 131.053664 102.22794) (end 119.195425 102.22794) (width 0.5) (layer "F.Cu") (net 19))
 (segment (start 119.192735 102.22525) (end 115.520933 102.22525) (width 0.5) (layer "F.Cu") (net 19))
 (segment (start 131.053664 102.22794) (end 134.665798 102.22794) (width 0.5) (layer "F.Cu") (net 19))
 (segment (start 119.187485 104.76) (end 119.182235 104.76525) (width 0.5) (layer "F.Cu") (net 20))
 (segment (start 119.182235 104.76525) (end 115.520933 104.76525) (width 0.5) (layer "F.Cu") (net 20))
 (segment (start 131.053664 104.76794) (end 134.665798 104.76794) (width 0.5) (layer "F.Cu") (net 20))
 (segment (start 119.187485 104.76) (end 131.045724 104.76) (width 0.5) (layer "F.Cu") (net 20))
 (segment (start 149.906902 56.509044) (end 161.88514 56.509044) (width 0.5) (layer "F.Cu") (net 40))
 (segment (start 146.293664 56.50794) (end 149.905798 56.50794) (width 0.5) (layer "F.Cu") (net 40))
 (segment (start 146.293664 59.04794) (end 149.905798 59.04794) (width 0.5) (layer "F.Cu") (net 39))
 (segment (start 149.906902 59.049044) (end 161.88514 59.049044) (width 0.5) (layer "F.Cu") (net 39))
 (segment (start 149.906902 61.589044) (end 161.88514 61.589044) (width 0.5) (layer "F.Cu") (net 38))
 (segment (start 146.293664 61.58794) (end 149.905798 61.58794) (width 0.5) (layer "F.Cu") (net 38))
 (segment (start 149.906902 64.129044) (end 161.88514 64.129044) (width 0.5) (layer "F.Cu") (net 37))
 (segment (start 146.293664 64.12794) (end 149.905798 64.12794) (width 0.5) (layer "F.Cu") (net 37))
 (segment (start 146.293664 66.66794) (end 149.905798 66.66794) (width 0.5) (layer "F.Cu") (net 36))
 (segment (start 149.906902 66.669044) (end 161.88514 66.669044) (width 0.5) (layer "F.Cu") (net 36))
 (segment (start 146.293664 69.20794) (end 149.905798 69.20794) (width 0.5) (layer "F.Cu") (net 35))
 (segment (start 149.906902 69.209044) (end 161.88514 69.209044) (width 0.5) (layer "F.Cu") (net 35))
 (segment (start 146.293664 71.74794) (end 149.905798 71.74794) (width 0.5) (layer "F.Cu") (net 34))
 (segment (start 149.906902 71.749044) (end 161.88514 71.749044) (width 0.5) (layer "F.Cu") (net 34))
 (segment (start 146.293664 74.28794) (end 149.905798 74.28794) (width 0.5) (layer "F.Cu") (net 33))
 (segment (start 149.906902 74.289044) (end 161.88514 74.289044) (width 0.5) (layer "F.Cu") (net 33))
 (segment (start 146.293664 76.82794) (end 149.905798 76.82794) (width 0.5) (layer "F.Cu") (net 32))
 (segment (start 149.906902 76.829044) (end 161.88514 76.829044) (width 0.5) (layer "F.Cu") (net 32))
 (segment (start 146.293664 79.36794) (end 149.905798 79.36794) (width 0.5) (layer "F.Cu") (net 31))
 (segment (start 149.906902 79.369044) (end 161.88514 79.369044) (width 0.5) (layer "F.Cu") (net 31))
 (segment (start 149.906902 81.909044) (end 161.88514 81.909044) (width 0.5) (layer "F.Cu") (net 30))
 (segment (start 146.293664 81.90794) (end 149.905798 81.90794) (width 0.5) (layer "F.Cu") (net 30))
 (segment (start 146.293664 86.98794) (end 149.905798 86.98794) (width 0.5) (layer "F.Cu") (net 28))
 (segment (start 149.906902 86.989044) (end 161.88514 86.989044) (width 0.5) (layer "F.Cu") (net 28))
 (segment (start 146.293664 89.52794) (end 149.905798 89.52794) (width 0.5) (layer "F.Cu") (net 27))
 (segment (start 149.906902 89.529044) (end 161.88514 89.529044) (width 0.5) (layer "F.Cu") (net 27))
 (segment (start 146.293664 92.06794) (end 149.905798 92.06794) (width 0.5) (layer "F.Cu") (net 26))
 (segment (start 149.906902 92.069044) (end 161.88514 92.069044) (width 0.5) (layer "F.Cu") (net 26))
 (segment (start 149.906902 94.609044) (end 161.88514 94.609044) (width 0.5) (layer "F.Cu") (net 25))
 (segment (start 146.293664 94.60794) (end 149.905798 94.60794) (width 0.5) (layer "F.Cu") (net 25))
 (segment (start 149.906902 97.149044) (end 161.88514 97.149044) (width 0.5) (layer "F.Cu") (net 24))
 (segment (start 146.293664 97.14794) (end 149.905798 97.14794) (width 0.5) (layer "F.Cu") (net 24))
 (segment (start 146.293664 99.68794) (end 149.905798 99.68794) (width 0.5) (layer "F.Cu") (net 23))
 (segment (start 149.906902 99.689044) (end 161.88514 99.689044) (width 0.5) (layer "F.Cu") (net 23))
 (segment (start 146.293664 102.22794) (end 149.905798 102.22794) (width 0.5) (layer "F.Cu") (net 22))
 (segment (start 149.906902 102.229044) (end 161.88514 102.229044) (width 0.5) (layer "F.Cu") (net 22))
 (segment (start 149.906902 104.769044) (end 161.88514 104.769044) (width 0.5) (layer "F.Cu") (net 21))
 (segment (start 146.293664 104.76794) (end 149.905798 104.76794) (width 0.5) (layer "F.Cu") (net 21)))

